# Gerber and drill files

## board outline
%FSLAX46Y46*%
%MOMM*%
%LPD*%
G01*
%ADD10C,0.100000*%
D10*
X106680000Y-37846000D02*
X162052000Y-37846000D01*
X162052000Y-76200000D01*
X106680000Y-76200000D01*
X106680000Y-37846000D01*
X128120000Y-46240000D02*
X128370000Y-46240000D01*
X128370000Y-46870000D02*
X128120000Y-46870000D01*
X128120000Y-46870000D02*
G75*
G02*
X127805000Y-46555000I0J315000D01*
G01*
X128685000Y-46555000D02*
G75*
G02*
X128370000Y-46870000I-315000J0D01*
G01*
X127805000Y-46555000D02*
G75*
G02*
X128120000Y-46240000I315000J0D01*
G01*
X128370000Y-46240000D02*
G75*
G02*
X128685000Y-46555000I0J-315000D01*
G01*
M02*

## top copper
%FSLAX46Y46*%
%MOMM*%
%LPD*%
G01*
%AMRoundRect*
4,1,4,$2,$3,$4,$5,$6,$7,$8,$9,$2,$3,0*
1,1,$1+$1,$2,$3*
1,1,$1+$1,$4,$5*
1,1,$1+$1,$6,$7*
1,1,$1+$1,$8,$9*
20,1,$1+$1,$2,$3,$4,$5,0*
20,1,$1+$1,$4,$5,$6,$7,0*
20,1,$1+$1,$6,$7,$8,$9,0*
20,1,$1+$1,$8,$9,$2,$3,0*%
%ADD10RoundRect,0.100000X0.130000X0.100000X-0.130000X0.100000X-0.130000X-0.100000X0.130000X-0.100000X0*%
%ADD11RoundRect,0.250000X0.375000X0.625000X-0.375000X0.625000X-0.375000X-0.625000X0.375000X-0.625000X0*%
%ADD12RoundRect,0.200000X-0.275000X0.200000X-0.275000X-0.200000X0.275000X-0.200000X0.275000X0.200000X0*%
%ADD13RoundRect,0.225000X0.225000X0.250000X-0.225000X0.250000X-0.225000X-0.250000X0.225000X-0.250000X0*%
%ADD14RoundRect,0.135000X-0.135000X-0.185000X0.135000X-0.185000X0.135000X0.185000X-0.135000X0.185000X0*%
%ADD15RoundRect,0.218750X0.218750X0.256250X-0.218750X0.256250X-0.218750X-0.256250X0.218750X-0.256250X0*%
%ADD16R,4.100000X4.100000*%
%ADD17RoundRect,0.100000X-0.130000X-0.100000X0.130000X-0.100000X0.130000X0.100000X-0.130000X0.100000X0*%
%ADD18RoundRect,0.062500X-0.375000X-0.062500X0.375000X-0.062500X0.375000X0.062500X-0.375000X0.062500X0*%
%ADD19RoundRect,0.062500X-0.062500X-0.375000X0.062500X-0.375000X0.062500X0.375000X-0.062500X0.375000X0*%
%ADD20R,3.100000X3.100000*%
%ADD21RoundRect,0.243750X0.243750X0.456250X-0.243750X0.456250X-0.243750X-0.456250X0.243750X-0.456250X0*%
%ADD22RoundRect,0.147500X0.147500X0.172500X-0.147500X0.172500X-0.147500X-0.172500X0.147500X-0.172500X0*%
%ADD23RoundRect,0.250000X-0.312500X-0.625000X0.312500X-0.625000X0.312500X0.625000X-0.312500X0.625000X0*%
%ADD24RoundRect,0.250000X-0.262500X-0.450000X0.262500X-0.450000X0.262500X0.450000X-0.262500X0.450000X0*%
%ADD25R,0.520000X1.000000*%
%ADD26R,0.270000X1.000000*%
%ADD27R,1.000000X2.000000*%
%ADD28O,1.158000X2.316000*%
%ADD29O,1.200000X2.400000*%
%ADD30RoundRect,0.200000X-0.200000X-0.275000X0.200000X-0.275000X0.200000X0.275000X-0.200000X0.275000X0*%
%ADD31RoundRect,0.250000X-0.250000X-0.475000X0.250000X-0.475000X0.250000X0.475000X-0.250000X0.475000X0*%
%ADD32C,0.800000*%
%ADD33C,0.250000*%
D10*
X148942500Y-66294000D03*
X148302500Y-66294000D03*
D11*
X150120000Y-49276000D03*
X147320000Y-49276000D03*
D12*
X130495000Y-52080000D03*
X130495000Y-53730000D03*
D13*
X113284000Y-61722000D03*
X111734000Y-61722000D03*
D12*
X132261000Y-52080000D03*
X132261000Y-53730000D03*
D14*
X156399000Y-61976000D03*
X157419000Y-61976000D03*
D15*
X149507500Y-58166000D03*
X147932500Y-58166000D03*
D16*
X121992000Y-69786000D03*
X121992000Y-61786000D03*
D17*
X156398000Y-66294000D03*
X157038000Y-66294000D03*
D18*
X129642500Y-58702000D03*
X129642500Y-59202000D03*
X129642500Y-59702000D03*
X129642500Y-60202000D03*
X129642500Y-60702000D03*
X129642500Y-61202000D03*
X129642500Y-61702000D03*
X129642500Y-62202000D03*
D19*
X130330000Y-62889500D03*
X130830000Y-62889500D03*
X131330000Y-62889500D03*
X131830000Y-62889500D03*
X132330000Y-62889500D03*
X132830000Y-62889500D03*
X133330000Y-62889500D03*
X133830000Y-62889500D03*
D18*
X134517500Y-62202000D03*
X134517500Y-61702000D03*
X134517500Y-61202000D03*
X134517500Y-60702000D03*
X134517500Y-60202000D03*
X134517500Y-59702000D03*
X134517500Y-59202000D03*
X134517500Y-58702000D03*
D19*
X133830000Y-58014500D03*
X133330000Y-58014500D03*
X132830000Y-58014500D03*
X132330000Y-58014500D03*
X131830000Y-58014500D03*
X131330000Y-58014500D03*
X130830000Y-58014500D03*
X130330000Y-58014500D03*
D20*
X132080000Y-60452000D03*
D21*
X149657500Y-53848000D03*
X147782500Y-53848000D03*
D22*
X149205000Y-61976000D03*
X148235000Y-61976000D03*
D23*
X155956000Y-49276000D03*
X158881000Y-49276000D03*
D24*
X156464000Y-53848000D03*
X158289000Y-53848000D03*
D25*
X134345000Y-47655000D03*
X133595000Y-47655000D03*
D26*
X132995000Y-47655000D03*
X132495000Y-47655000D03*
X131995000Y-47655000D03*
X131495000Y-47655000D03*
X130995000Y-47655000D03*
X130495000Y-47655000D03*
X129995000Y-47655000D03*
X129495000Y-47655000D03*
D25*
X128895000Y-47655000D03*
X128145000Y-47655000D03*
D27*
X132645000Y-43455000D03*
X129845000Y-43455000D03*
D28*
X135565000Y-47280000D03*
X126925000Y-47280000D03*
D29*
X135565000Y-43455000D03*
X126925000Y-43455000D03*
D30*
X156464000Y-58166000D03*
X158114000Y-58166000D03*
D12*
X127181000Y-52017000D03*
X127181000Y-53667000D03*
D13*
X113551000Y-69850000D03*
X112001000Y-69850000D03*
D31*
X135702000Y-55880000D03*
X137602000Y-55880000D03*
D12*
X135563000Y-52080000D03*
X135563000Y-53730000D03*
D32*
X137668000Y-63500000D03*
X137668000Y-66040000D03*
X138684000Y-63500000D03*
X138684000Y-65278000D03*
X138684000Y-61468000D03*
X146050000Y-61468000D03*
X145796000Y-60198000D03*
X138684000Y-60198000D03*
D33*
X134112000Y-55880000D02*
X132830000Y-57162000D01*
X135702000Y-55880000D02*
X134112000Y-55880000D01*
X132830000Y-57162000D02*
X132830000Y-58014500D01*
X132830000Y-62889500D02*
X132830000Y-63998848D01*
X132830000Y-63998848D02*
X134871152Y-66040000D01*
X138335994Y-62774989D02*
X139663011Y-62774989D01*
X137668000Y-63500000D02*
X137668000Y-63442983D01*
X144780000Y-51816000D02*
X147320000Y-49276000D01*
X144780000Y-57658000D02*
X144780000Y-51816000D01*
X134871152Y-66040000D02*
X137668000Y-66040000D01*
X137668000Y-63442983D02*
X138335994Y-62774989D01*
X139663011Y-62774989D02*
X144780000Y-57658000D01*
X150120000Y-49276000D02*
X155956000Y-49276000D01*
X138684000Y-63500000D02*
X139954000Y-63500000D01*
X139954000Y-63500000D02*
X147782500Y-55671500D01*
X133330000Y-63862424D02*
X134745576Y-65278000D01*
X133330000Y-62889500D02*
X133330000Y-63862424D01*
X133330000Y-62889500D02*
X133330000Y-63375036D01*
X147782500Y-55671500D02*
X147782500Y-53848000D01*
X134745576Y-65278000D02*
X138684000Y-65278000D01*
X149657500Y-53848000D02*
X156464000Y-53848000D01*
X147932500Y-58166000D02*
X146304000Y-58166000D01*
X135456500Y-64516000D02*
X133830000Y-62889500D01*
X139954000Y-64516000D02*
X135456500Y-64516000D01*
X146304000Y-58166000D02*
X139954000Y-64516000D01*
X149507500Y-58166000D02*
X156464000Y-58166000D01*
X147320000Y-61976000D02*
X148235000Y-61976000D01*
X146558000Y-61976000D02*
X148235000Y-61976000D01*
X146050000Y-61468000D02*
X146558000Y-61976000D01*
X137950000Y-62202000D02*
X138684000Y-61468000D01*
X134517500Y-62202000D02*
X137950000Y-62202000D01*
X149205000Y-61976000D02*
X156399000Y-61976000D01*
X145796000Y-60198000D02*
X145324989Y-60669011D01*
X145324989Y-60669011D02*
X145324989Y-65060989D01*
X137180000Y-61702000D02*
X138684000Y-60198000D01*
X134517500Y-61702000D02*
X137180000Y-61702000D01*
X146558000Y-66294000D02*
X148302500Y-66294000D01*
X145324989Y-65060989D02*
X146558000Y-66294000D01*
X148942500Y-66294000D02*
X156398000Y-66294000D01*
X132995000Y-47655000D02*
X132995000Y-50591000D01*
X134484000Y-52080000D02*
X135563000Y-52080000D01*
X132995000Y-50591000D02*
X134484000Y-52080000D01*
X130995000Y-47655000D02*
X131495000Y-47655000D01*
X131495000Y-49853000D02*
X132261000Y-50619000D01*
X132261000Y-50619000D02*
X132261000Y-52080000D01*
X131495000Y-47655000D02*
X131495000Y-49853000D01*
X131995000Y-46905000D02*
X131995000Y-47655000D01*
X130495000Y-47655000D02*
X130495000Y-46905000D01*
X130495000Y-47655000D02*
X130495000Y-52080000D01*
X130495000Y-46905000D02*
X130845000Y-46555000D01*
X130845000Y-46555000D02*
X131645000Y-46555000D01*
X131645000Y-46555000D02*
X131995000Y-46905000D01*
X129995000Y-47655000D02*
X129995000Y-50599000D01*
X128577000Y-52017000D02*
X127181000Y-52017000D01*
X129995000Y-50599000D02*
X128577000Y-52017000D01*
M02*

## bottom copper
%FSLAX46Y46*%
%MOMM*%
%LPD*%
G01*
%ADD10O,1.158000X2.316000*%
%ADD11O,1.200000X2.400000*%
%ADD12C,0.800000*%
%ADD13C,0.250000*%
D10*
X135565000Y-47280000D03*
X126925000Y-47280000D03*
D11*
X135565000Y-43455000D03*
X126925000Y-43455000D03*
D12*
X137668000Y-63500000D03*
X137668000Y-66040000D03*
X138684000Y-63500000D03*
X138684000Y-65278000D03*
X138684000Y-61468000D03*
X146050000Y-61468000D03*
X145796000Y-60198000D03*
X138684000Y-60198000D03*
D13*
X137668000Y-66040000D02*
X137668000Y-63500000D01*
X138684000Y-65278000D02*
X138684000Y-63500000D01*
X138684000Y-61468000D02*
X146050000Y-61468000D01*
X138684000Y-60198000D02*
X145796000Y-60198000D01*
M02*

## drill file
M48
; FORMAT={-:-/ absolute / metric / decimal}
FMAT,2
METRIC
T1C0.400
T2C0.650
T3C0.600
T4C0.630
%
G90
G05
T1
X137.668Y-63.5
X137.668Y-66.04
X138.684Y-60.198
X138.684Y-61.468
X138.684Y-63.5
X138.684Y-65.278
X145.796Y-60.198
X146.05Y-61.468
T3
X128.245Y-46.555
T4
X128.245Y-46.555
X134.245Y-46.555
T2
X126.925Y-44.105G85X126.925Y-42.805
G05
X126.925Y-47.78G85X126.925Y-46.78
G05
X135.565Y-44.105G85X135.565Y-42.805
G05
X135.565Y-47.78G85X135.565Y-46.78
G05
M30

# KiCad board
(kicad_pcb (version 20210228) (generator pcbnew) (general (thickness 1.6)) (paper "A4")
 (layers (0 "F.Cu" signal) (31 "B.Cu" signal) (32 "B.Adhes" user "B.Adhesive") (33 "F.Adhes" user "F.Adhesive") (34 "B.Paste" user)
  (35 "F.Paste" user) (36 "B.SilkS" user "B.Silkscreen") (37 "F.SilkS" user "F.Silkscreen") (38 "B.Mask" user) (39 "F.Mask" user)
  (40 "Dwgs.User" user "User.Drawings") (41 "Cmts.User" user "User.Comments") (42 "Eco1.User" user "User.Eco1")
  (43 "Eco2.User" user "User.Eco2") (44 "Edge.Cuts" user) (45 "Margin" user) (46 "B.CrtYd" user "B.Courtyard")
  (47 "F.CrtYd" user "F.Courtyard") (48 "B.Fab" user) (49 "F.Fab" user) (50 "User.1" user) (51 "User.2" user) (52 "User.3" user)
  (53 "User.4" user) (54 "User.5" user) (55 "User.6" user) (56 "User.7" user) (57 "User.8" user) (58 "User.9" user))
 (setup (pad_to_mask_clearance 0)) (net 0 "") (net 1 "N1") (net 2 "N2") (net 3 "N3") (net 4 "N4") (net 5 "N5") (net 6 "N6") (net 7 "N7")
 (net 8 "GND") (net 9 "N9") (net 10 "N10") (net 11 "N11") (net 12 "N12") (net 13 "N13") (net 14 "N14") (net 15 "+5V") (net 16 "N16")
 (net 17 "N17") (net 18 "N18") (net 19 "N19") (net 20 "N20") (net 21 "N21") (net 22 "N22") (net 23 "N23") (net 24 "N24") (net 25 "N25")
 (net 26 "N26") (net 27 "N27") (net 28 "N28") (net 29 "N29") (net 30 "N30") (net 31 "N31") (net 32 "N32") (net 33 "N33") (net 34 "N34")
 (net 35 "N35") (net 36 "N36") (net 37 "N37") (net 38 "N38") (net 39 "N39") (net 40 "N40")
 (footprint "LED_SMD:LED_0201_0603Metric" (layer "F.Cu") (at 148.6225 66.294 180)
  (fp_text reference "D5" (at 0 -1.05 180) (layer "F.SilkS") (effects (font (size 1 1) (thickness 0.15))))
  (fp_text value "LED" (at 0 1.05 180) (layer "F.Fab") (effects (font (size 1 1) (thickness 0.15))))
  (pad "" smd roundrect (at 0.345 0 180) (locked) (size 0.318 0.36) (layers "F.Paste") (roundrect_rratio 0.25))
  (pad "" smd roundrect (at -0.345 0 180) (locked) (size 0.318 0.36) (layers "F.Paste") (roundrect_rratio 0.25))
  (pad "1" smd roundrect (at -0.32 0 180) (locked) (size 0.46 0.4) (layers "F.Cu" "F.Mask") (roundrect_rratio 0.25) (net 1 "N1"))
  (pad "2" smd roundrect (at 0.32 0 180) (locked) (size 0.46 0.4) (layers "F.Cu" "F.Mask") (roundrect_rratio 0.25) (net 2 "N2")))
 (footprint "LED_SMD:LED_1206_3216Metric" (layer "F.Cu") (at 148.72 49.276 180)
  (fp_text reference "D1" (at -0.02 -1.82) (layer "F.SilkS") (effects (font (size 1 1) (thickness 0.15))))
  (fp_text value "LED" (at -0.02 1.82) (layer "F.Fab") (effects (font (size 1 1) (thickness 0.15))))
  (pad "1" smd roundrect (at -1.4 0 180) (locked) (size 1.25 1.75) (layers "F.Cu" "F.Paste" "F.Mask") (roundrect_rratio 0.2) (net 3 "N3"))
  (pad "2" smd roundrect (at 1.4 0 180) (locked) (size 1.25 1.75) (layers "F.Cu" "F.Paste" "F.Mask") (roundrect_rratio 0.2) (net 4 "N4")))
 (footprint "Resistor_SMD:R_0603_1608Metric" (layer "F.Cu") (at 130.495 52.905 -90)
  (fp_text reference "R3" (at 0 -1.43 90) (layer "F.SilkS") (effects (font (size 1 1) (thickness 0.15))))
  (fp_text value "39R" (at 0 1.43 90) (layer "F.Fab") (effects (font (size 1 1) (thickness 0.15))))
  (pad "1" smd roundrect (at -0.825 0 270) (locked) (size 0.8 0.95) (layers "F.Cu" "F.Paste" "F.Mask") (roundrect_rratio 0.25) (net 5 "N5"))
  (pad "2" smd roundrect (at 0.825 0 270) (locked) (size 0.8 0.95) (layers "F.Cu" "F.Paste" "F.Mask") (roundrect_rratio 0.25) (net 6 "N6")))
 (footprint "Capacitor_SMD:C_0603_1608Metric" (layer "F.Cu") (at 112.509 61.722 180)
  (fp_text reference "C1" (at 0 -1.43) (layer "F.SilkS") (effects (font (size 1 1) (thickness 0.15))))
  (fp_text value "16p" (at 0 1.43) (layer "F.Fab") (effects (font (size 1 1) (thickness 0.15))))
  (pad "1" smd roundrect (at -0.775 0 180) (locked) (size 0.9 0.95) (layers "F.Cu" "F.Paste" "F.Mask") (roundrect_rratio 0.25) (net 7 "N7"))
  (pad "2" smd roundrect (at 0.775 0 180) (locked) (size 0.9 0.95) (layers "F.Cu" "F.Paste" "F.Mask") (roundrect_rratio 0.25) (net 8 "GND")))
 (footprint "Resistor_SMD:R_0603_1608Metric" (layer "F.Cu") (at 132.261 52.905 -90)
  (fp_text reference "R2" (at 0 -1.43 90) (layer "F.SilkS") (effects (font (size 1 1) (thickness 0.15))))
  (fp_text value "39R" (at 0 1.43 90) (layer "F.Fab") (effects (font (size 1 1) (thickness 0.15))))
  (pad "1" smd roundrect (at -0.825 0 270) (locked) (size 0.8 0.95) (layers "F.Cu" "F.Paste" "F.Mask") (roundrect_rratio 0.25) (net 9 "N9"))
  (pad "2" smd roundrect (at 0.825 0 270) (locked) (size 0.8 0.95) (layers "F.Cu" "F.Paste" "F.Mask") (roundrect_rratio 0.25) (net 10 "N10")))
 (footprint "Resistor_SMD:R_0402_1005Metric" (layer "F.Cu") (at 156.909 61.976)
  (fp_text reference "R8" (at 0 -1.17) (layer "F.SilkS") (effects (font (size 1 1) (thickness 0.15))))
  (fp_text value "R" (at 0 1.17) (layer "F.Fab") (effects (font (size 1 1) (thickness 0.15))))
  (pad "1" smd roundrect (at -0.51 0) (locked) (size 0.54 0.64) (layers "F.Cu" "F.Paste" "F.Mask") (roundrect_rratio 0.25) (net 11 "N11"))
  (pad "2" smd roundrect (at 0.51 0) (locked) (size 0.54 0.64) (layers "F.Cu" "F.Paste" "F.Mask") (roundrect_rratio 0.25) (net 8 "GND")))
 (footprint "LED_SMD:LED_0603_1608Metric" (layer "F.Cu") (at 148.72 58.166 180)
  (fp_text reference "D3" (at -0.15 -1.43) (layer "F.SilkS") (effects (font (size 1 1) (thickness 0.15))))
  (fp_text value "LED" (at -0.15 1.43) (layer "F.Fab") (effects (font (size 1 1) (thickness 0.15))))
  (pad "1" smd roundrect (at -0.7875 0 180) (locked) (size 0.875 0.95) (layers "F.Cu" "F.Paste" "F.Mask") (roundrect_rratio 0.25)
   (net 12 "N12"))
  (pad "2" smd roundrect (at 0.7875 0 180) (locked) (size 0.875 0.95) (layers "F.Cu" "F.Paste" "F.Mask") (roundrect_rratio 0.25)
   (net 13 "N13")))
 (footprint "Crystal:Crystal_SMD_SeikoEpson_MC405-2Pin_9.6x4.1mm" (layer "F.Cu") (at 121.992 65.786 90)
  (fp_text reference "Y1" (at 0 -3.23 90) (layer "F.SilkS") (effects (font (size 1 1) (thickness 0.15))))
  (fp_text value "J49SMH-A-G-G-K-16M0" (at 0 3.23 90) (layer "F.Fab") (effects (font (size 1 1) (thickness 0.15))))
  (pad "1" smd rect (at -4 0 90) (locked) (size 4.1 4.1) (layers "F.Cu" "F.Paste" "F.Mask") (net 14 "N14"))
  (pad "2" smd rect (at 4 0 90) (locked) (size 4.1 4.1) (layers "F.Cu" "F.Paste" "F.Mask") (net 7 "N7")))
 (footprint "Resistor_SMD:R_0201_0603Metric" (layer "F.Cu") (at 156.718 66.294)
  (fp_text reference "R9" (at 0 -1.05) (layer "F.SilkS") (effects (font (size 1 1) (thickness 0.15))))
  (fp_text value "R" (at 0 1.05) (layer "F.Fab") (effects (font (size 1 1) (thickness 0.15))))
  (pad "" smd roundrect (at -0.345 0) (locked) (size 0.318 0.36) (layers "F.Paste") (roundrect_rratio 0.25))
  (pad "" smd roundrect (at 0.345 0) (locked) (size 0.318 0.36) (layers "F.Paste") (roundrect_rratio 0.25))
  (pad "1" smd roundrect (at -0.32 0) (locked) (size 0.46 0.4) (layers "F.Cu" "F.Mask") (roundrect_rratio 0.25) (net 1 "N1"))
  (pad "2" smd roundrect (at 0.32 0) (locked) (size 0.46 0.4) (layers "F.Cu" "F.Mask") (roundrect_rratio 0.25) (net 8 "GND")))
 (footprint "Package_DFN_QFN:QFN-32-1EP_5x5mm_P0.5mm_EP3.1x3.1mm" (layer "F.Cu") (at 132.08 60.452)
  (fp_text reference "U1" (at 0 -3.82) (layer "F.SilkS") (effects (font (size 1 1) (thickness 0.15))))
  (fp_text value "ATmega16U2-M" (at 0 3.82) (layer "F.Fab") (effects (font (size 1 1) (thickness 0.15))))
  (pad "" smd roundrect (at 1.03 -1.03) (locked) (size 0.83 0.83) (layers "F.Paste") (roundrect_rratio 0.25))
  (pad "" smd roundrect (at 0 -1.03) (locked) (size 0.83 0.83) (layers "F.Paste") (roundrect_rratio 0.25))
  (pad "" smd roundrect (at 0 1.03) (locked) (size 0.83 0.83) (layers "F.Paste") (roundrect_rratio 0.25))
  (pad "" smd roundrect (at 0 0) (locked) (size 0.83 0.83) (layers "F.Paste") (roundrect_rratio 0.25))
  (pad "" smd roundrect (at 1.03 1.03) (locked) (size 0.83 0.83) (layers "F.Paste") (roundrect_rratio 0.25))
  (pad "" smd roundrect (at 1.03 0) (locked) (size 0.83 0.83) (layers "F.Paste") (roundrect_rratio 0.25))
  (pad "" smd roundrect (at -1.03 -1.03) (locked) (size 0.83 0.83) (layers "F.Paste") (roundrect_rratio 0.25))
  (pad "" smd roundrect (at -1.03 1.03) (locked) (size 0.83 0.83) (layers "F.Paste") (roundrect_rratio 0.25))
  (pad "" smd roundrect (at -1.03 0) (locked) (size 0.83 0.83) (layers "F.Paste") (roundrect_rratio 0.25))
  (pad "1" smd roundrect (at -2.4375 -1.75) (locked) (size 0.875 0.25) (layers "F.Cu" "F.Paste" "F.Mask") (roundrect_rratio 0.25)
   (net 7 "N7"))
  (pad "2" smd roundrect (at -2.4375 -1.25) (locked) (size 0.875 0.25) (layers "F.Cu" "F.Paste" "F.Mask") (roundrect_rratio 0.25)
   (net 14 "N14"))
  (pad "3" smd roundrect (at -2.4375 -0.75) (locked) (size 0.875 0.25) (layers "F.Cu" "F.Paste" "F.Mask") (roundrect_rratio 0.25)
   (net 8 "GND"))
  (pad "4" smd roundrect (at -2.4375 -0.25) (locked) (size 0.875 0.25) (layers "F.Cu" "F.Paste" "F.Mask") (roundrect_rratio 0.25)
   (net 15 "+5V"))
  (pad "5" smd roundrect (at -2.4375 0.25) (locked) (size 0.875 0.25) (layers "F.Cu" "F.Paste" "F.Mask") (roundrect_rratio 0.25)
   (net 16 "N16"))
  (pad "6" smd roundrect (at -2.4375 0.75) (locked) (size 0.875 0.25) (layers "F.Cu" "F.Paste" "F.Mask") (roundrect_rratio 0.25)
   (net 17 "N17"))
  (pad "7" smd roundrect (at -2.4375 1.25) (locked) (size 0.875 0.25) (layers "F.Cu" "F.Paste" "F.Mask") (roundrect_rratio 0.25)
   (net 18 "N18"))
  (pad "8" smd roundrect (at -2.4375 1.75) (locked) (size 0.875 0.25) (layers "F.Cu" "F.Paste" "F.Mask") (roundrect_rratio 0.25)
   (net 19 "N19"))
  (pad "9" smd roundrect (at -1.75 2.4375) (locked) (size 0.25 0.875) (layers "F.Cu" "F.Paste" "F.Mask") (roundrect_rratio 0.25)
   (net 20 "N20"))
  (pad "10" smd roundrect (at -1.25 2.4375) (locked) (size 0.25 0.875) (layers "F.Cu" "F.Paste" "F.Mask") (roundrect_rratio 0.25)
   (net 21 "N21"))
  (pad "11" smd roundrect (at -0.75 2.4375) (locked) (size 0.25 0.875) (layers "F.Cu" "F.Paste" "F.Mask") (roundrect_rratio 0.25)
   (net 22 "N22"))
  (pad "12" smd roundrect (at -0.25 2.4375) (locked) (size 0.25 0.875) (layers "F.Cu" "F.Paste" "F.Mask") (roundrect_rratio 0.25)
   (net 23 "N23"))
  (pad "13" smd roundrect (at 0.25 2.4375) (locked) (size 0.25 0.875) (layers "F.Cu" "F.Paste" "F.Mask") (roundrect_rratio 0.25)
   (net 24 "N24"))
  (pad "14" smd roundrect (at 0.75 2.4375) (locked) (size 0.25 0.875) (layers "F.Cu" "F.Paste" "F.Mask") (roundrect_rratio 0.25)
   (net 4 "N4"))
  (pad "15" smd roundrect (at 1.25 2.4375) (locked) (size 0.25 0.875) (layers "F.Cu" "F.Paste" "F.Mask") (roundrect_rratio 0.25)
   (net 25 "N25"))
  (pad "16" smd roundrect (at 1.75 2.4375) (locked) (size 0.25 0.875) (layers "F.Cu" "F.Paste" "F.Mask") (roundrect_rratio 0.25)
   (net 13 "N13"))
  (pad "17" smd roundrect (at 2.4375 1.75) (locked) (size 0.875 0.25) (layers "F.Cu" "F.Paste" "F.Mask") (roundrect_rratio 0.25)
   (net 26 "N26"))
  (pad "18" smd roundrect (at 2.4375 1.25) (locked) (size 0.875 0.25) (layers "F.Cu" "F.Paste" "F.Mask") (roundrect_rratio 0.25)
   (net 2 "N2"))
  (pad "19" smd roundrect (at 2.4375 0.75) (locked) (size 0.875 0.25) (layers "F.Cu" "F.Paste" "F.Mask") (roundrect_rratio 0.25)
   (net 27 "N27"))
  (pad "20" smd roundrect (at 2.4375 0.25) (locked) (size 0.875 0.25) (layers "F.Cu" "F.Paste" "F.Mask") (roundrect_rratio 0.25)
   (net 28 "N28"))
  (pad "21" smd roundrect (at 2.4375 -0.25) (locked) (size 0.875 0.25) (layers "F.Cu" "F.Paste" "F.Mask") (roundrect_rratio 0.25)
   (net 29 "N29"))
  (pad "22" smd roundrect (at 2.4375 -0.75) (locked) (size 0.875 0.25) (layers "F.Cu" "F.Paste" "F.Mask") (roundrect_rratio 0.25)
   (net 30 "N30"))
  (pad "23" smd roundrect (at 2.4375 -1.25) (locked) (size 0.875 0.25) (layers "F.Cu" "F.Paste" "F.Mask") (roundrect_rratio 0.25)
   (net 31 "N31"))
  (pad "24" smd roundrect (at 2.4375 -1.75) (locked) (size 0.875 0.25) (layers "F.Cu" "F.Paste" "F.Mask") (roundrect_rratio 0.25)
   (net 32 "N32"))
  (pad "25" smd roundrect (at 1.75 -2.4375) (locked) (size 0.25 0.875) (layers "F.Cu" "F.Paste" "F.Mask") (roundrect_rratio 0.25)
   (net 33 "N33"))
  (pad "26" smd roundrect (at 1.25 -2.4375) (locked) (size 0.25 0.875) (layers "F.Cu" "F.Paste" "F.Mask") (roundrect_rratio 0.25)
   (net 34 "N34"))
  (pad "27" smd roundrect (at 0.75 -2.4375) (locked) (size 0.25 0.875) (layers "F.Cu" "F.Paste" "F.Mask") (roundrect_rratio 0.25)
   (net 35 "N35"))
  (pad "28" smd roundrect (at 0.25 -2.4375) (locked) (size 0.25 0.875) (layers "F.Cu" "F.Paste" "F.Mask") (roundrect_rratio 0.25)
   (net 8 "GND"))
  (pad "29" smd roundrect (at -0.25 -2.4375) (locked) (size 0.25 0.875) (layers "F.Cu" "F.Paste" "F.Mask") (roundrect_rratio 0.25)
   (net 10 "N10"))
  (pad "30" smd roundrect (at -0.75 -2.4375) (locked) (size 0.25 0.875) (layers "F.Cu" "F.Paste" "F.Mask") (roundrect_rratio 0.25)
   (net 6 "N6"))
  (pad "31" smd roundrect (at -1.25 -2.4375) (locked) (size 0.25 0.875) (layers "F.Cu" "F.Paste" "F.Mask") (roundrect_rratio 0.25)
   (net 15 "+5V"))
  (pad "32" smd roundrect (at -1.75 -2.4375) (locked) (size 0.25 0.875) (layers "F.Cu" "F.Paste" "F.Mask") (roundrect_rratio 0.25)
   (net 15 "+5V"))
  (pad "33" smd rect (at 0 0) (locked) (size 3.1 3.1) (layers "F.Cu" "F.Mask") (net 8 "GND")))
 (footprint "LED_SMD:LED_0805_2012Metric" (layer "F.Cu") (at 148.72 53.848 180)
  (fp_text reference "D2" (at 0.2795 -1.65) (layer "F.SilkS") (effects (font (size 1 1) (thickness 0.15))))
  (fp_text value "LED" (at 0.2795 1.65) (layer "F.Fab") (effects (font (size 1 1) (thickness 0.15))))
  (pad "1" smd roundrect (at -0.9375 0 180) (locked) (size 0.975 1.4) (layers "F.Cu" "F.Paste" "F.Mask") (roundrect_rratio 0.25)
   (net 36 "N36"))
  (pad "2" smd roundrect (at 0.9375 0 180) (locked) (size 0.975 1.4) (layers "F.Cu" "F.Paste" "F.Mask") (roundrect_rratio 0.25)
   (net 25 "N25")))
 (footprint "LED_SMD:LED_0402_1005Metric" (layer "F.Cu") (at 148.72 61.976 180)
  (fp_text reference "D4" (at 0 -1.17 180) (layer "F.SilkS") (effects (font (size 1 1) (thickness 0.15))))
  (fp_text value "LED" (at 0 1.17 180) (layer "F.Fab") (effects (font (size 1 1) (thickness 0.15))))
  (pad "1" smd roundrect (at -0.485 0 180) (locked) (size 0.59 0.64) (layers "F.Cu" "F.Paste" "F.Mask") (roundrect_rratio 0.25)
   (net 11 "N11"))
  (pad "2" smd roundrect (at 0.485 0 180) (locked) (size 0.59 0.64) (layers "F.Cu" "F.Paste" "F.Mask") (roundrect_rratio 0.25)
   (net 26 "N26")))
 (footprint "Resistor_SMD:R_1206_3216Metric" (layer "F.Cu") (at 157.4185 49.276)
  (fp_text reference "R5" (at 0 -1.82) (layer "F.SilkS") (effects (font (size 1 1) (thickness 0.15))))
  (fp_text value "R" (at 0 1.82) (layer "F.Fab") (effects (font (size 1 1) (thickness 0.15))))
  (pad "1" smd roundrect (at -1.4625 0) (locked) (size 1.125 1.75) (layers "F.Cu" "F.Paste" "F.Mask") (roundrect_rratio 0.222222)
   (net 3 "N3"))
  (pad "2" smd roundrect (at 1.4625 0) (locked) (size 1.125 1.75) (layers "F.Cu" "F.Paste" "F.Mask") (roundrect_rratio 0.222222)
   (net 8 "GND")))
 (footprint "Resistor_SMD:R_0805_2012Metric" (layer "F.Cu") (at 157.3765 53.848)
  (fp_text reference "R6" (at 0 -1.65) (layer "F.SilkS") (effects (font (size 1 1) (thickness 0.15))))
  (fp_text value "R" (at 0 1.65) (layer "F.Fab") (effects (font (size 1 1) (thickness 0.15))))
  (pad "1" smd roundrect (at -0.9125 0) (locked) (size 1.025 1.4) (layers "F.Cu" "F.Paste" "F.Mask") (roundrect_rratio 0.243902)
   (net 36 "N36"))
  (pad "2" smd roundrect (at 0.9125 0) (locked) (size 1.025 1.4) (layers "F.Cu" "F.Paste" "F.Mask") (roundrect_rratio 0.243902)
   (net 8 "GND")))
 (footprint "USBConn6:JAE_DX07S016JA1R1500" (layer "F.Cu") (at 131.245 46.555 180)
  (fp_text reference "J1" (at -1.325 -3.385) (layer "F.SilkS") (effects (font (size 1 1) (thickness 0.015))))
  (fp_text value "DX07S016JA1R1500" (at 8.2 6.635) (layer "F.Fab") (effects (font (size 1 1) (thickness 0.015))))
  (fp_line (start 3.125 0.315) (end 2.875 0.315) (layer "Edge.Cuts") (width 0.1))
  (fp_line (start 2.875 -0.315) (end 3.125 -0.315) (layer "Edge.Cuts") (width 0.1))
  (fp_arc (start 3.125 0) (end 3.44 0) (angle -90) (layer "Edge.Cuts") (width 0.1))
  (fp_arc (start 2.875 0) (end 2.875 -0.315) (angle -90) (layer "Edge.Cuts") (width 0.1))
  (fp_arc (start 3.125 0) (end 3.125 0.315) (angle -90) (layer "Edge.Cuts") (width 0.1))
  (fp_arc (start 2.875 0) (end 2.56 0) (angle -90) (layer "Edge.Cuts") (width 0.1))
  (pad "1" smd rect (at -3.1 -1.1 180) (locked) (size 0.52 1) (layers "F.Cu" "F.Paste" "F.Mask") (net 8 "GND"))
  (pad "2" smd rect (at -2.35 -1.1 180) (locked) (size 0.52 1) (layers "F.Cu" "F.Paste" "F.Mask") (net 15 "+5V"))
  (pad "3" smd rect (at -1.75 -1.1 180) (locked) (size 0.27 1) (layers "F.Cu" "F.Paste" "F.Mask") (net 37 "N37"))
  (pad "4" smd rect (at -1.25 -1.1 180) (locked) (size 0.27 1) (layers "F.Cu" "F.Paste" "F.Mask") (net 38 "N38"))
  (pad "5" smd rect (at -0.75 -1.1 180) (locked) (size 0.27 1) (layers "F.Cu" "F.Paste" "F.Mask") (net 5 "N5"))
  (pad "6" smd rect (at -0.25 -1.1 180) (locked) (size 0.27 1) (layers "F.Cu" "F.Paste" "F.Mask") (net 9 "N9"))
  (pad "7" smd rect (at 0.25 -1.1 180) (locked) (size 0.27 1) (layers "F.Cu" "F.Paste" "F.Mask") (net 9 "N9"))
  (pad "8" smd rect (at 0.75 -1.1 180) (locked) (size 0.27 1) (layers "F.Cu" "F.Paste" "F.Mask") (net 5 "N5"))
  (pad "9" smd rect (at 1.25 -1.1 180) (locked) (size 0.27 1) (layers "F.Cu" "F.Paste" "F.Mask") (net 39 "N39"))
  (pad "10" smd rect (at 1.75 -1.1 180) (locked) (size 0.27 1) (layers "F.Cu" "F.Paste" "F.Mask") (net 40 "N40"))
  (pad "11" smd rect (at 2.35 -1.1 180) (locked) (size 0.52 1) (layers "F.Cu" "F.Paste" "F.Mask") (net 15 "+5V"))
  (pad "12" smd rect (at 3.1 -1.1 180) (locked) (size 0.52 1) (layers "F.Cu" "F.Paste" "F.Mask") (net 8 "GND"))
  (pad "None" np_thru_hole circle (at 3 0 180) (locked) (size 0.63 0.63) (drill 0.63) (layers *.Cu *.Mask))
  (pad "None" np_thru_hole circle (at 3 0 180) (locked) (size 0.6 0.6) (drill 0.6) (layers *.Cu *.Mask))
  (pad "None" np_thru_hole circle (at -3 0 180) (locked) (size 0.63 0.63) (drill 0.63) (layers *.Cu *.Mask))
  (pad "S1" smd rect (at -1.4 3.1 180) (locked) (size 1 2) (layers "F.Cu" "F.Paste" "F.Mask") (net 8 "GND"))
  (pad "S2" smd rect (at 1.4 3.1 180) (locked) (size 1 2) (layers "F.Cu" "F.Paste" "F.Mask") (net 8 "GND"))
  (pad "S3" thru_hole oval (at -4.32 -0.725 180) (locked) (size 1.158 2.316) (drill oval 0.65 1.65) (layers *.Cu *.Mask) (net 8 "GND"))
  (pad "S4" thru_hole oval (at 4.32 -0.725 180) (locked) (size 1.158 2.316) (drill oval 0.65 1.65) (layers *.Cu *.Mask) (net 8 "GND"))
  (pad "S5" thru_hole oval (at -4.32 3.1 180) (locked) (size 1.2 2.4) (drill oval 0.65 1.95) (layers *.Cu *.Mask) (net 8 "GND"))
  (pad "S6" thru_hole oval (at 4.32 3.1 180) (locked) (size 1.2 2.4) (drill oval 0.65 1.95) (layers *.Cu *.Mask) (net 8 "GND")))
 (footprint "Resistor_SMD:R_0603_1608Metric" (layer "F.Cu") (at 157.289 58.166)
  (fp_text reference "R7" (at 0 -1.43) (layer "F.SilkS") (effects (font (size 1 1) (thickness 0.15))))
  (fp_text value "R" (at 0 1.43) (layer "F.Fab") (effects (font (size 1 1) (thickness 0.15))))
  (pad "1" smd roundrect (at -0.825 0) (locked) (size 0.8 0.95) (layers "F.Cu" "F.Paste" "F.Mask") (roundrect_rratio 0.25) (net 12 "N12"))
  (pad "2" smd roundrect (at 0.825 0) (locked) (size 0.8 0.95) (layers "F.Cu" "F.Paste" "F.Mask") (roundrect_rratio 0.25) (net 8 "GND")))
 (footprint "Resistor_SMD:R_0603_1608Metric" (layer "F.Cu") (at 127.181 52.842 -90)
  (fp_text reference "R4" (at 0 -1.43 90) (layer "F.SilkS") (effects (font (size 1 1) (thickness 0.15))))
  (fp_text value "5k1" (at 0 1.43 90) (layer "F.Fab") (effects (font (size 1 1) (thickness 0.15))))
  (pad "1" smd roundrect (at -0.825 0 270) (locked) (size 0.8 0.95) (layers "F.Cu" "F.Paste" "F.Mask") (roundrect_rratio 0.25)
   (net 39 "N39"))
  (pad "2" smd roundrect (at 0.825 0 270) (locked) (size 0.8 0.95) (layers "F.Cu" "F.Paste" "F.Mask") (roundrect_rratio 0.25) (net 8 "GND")))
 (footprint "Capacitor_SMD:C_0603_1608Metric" (layer "F.Cu") (at 112.776 69.85 180)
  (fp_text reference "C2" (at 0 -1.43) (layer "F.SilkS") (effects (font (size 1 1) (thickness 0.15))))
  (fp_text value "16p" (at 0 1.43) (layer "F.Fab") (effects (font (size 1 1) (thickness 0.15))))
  (pad "1" smd roundrect (at -0.775 0 180) (locked) (size 0.9 0.95) (layers "F.Cu" "F.Paste" "F.Mask") (roundrect_rratio 0.25)
   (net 14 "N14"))
  (pad "2" smd roundrect (at 0.775 0 180) (locked) (size 0.9 0.95) (layers "F.Cu" "F.Paste" "F.Mask") (roundrect_rratio 0.25) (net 8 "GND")))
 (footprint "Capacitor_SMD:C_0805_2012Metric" (layer "F.Cu") (at 136.652 55.88)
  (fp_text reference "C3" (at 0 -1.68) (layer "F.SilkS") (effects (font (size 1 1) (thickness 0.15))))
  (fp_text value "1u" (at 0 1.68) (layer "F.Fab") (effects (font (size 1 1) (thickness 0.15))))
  (pad "1" smd roundrect (at -0.95 0) (locked) (size 1 1.45) (layers "F.Cu" "F.Paste" "F.Mask") (roundrect_rratio 0.25) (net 35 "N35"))
  (pad "2" smd roundrect (at 0.95 0) (locked) (size 1 1.45) (layers "F.Cu" "F.Paste" "F.Mask") (roundrect_rratio 0.25) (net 8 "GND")))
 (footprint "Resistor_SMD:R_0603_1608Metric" (layer "F.Cu") (at 135.563 52.905 -90)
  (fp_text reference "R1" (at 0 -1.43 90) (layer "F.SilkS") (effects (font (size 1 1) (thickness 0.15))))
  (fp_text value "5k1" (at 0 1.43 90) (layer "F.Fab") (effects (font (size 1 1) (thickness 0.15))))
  (pad "1" smd roundrect (at -0.825 0 270) (locked) (size 0.8 0.95) (layers "F.Cu" "F.Paste" "F.Mask") (roundrect_rratio 0.25)
   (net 37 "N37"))
  (pad "2" smd roundrect (at 0.825 0 270) (locked) (size 0.8 0.95) (layers "F.Cu" "F.Paste" "F.Mask") (roundrect_rratio 0.25) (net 8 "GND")))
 (gr_rect (start 106.68 37.846) (end 162.052 76.2) (layer "Edge.Cuts") (width 0.1) (fill none))
 (segment (start 134.112 55.88) (end 132.83 57.162) (width 0.25) (layer "F.Cu") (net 35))
 (segment (start 135.702 55.88) (end 134.112 55.88) (width 0.25) (layer "F.Cu") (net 35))
 (segment (start 132.83 57.162) (end 132.83 58.0145) (width 0.25) (layer "F.Cu") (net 35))
 (segment (start 132.83 62.8895) (end 132.83 63.998848) (width 0.25) (layer "F.Cu") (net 4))
 (segment (start 132.83 63.998848) (end 134.871152 66.04) (width 0.25) (layer "F.Cu") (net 4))
 (segment (start 138.335994 62.774989) (end 139.663011 62.774989) (width 0.25) (layer "F.Cu") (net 4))
 (segment (start 137.668 63.5) (end 137.668 63.442983) (width 0.25) (layer "F.Cu") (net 4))
 (segment (start 144.78 51.816) (end 147.32 49.276) (width 0.25) (layer "F.Cu") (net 4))
 (segment (start 144.78 57.658) (end 144.78 51.816) (width 0.25) (layer "F.Cu") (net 4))
 (segment (start 134.871152 66.04) (end 137.668 66.04) (width 0.25) (layer "F.Cu") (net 4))
 (segment (start 137.668 63.442983) (end 138.335994 62.774989) (width 0.25) (layer "F.Cu") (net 4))
 (segment (start 139.663011 62.774989) (end 144.78 57.658) (width 0.25) (layer "F.Cu") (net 4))
 (via (at 137.668 63.5) (size 0.8) (drill 0.4) (layers "F.Cu" "B.Cu") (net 4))
 (via (at 137.668 66.04) (size 0.8) (drill 0.4) (layers "F.Cu" "B.Cu") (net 4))
 (segment (start 137.668 66.04) (end 137.668 63.5) (width 0.25) (layer "B.Cu") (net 4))
 (segment (start 150.12 49.276) (end 155.956 49.276) (width 0.25) (layer "F.Cu") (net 3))
 (segment (start 138.684 63.5) (end 139.954 63.5) (width 0.25) (layer "F.Cu") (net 25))
 (segment (start 139.954 63.5) (end 147.7825 55.6715) (width 0.25) (layer "F.Cu") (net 25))
 (segment (start 133.33 63.862424) (end 134.745576 65.278) (width 0.25) (layer "F.Cu") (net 25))
 (segment (start 133.33 62.8895) (end 133.33 63.862424) (width 0.25) (layer "F.Cu") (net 25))
 (segment (start 133.33 62.8895) (end 133.33 63.375036) (width 0.25) (layer "F.Cu") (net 25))
 (segment (start 147.7825 55.6715) (end 147.7825 53.848) (width 0.25) (layer "F.Cu") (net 25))
 (segment (start 134.745576 65.278) (end 138.684 65.278) (width 0.25) (layer "F.Cu") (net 25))
 (via (at 138.684 63.5) (size 0.8) (drill 0.4) (layers "F.Cu" "B.Cu") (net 25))
 (via (at 138.684 65.278) (size 0.8) (drill 0.4) (layers "F.Cu" "B.Cu") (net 25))
 (segment (start 138.684 65.278) (end 138.684 63.5) (width 0.25) (layer "B.Cu") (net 25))
 (segment (start 149.6575 53.848) (end 156.464 53.848) (width 0.25) (layer "F.Cu") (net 36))
 (segment (start 147.9325 58.166) (end 146.304 58.166) (width 0.25) (layer "F.Cu") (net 13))
 (segment (start 135.4565 64.516) (end 133.83 62.8895) (width 0.25) (layer "F.Cu") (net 13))
 (segment (start 139.954 64.516) (end 135.4565 64.516) (width 0.25) (layer "F.Cu") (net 13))
 (segment (start 146.304 58.166) (end 139.954 64.516) (width 0.25) (layer "F.Cu") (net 13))
 (segment (start 149.5075 58.166) (end 156.464 58.166) (width 0.25) (layer "F.Cu") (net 12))
 (segment (start 147.32 61.976) (end 148.235 61.976) (width 0.25) (layer "F.Cu") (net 26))
 (segment (start 146.558 61.976) (end 148.235 61.976) (width 0.25) (layer "F.Cu") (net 26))
 (segment (start 146.05 61.468) (end 146.558 61.976) (width 0.25) (layer "F.Cu") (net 26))
 (segment (start 137.95 62.202) (end 138.684 61.468) (width 0.25) (layer "F.Cu") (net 26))
 (segment (start 134.5175 62.202) (end 137.95 62.202) (width 0.25) (layer "F.Cu") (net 26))
 (via (at 138.684 61.468) (size 0.8) (drill 0.4) (layers "F.Cu" "B.Cu") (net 26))
 (via (at 146.05 61.468) (size 0.8) (drill 0.4) (layers "F.Cu" "B.Cu") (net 26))
 (segment (start 138.684 61.468) (end 146.05 61.468) (width 0.25) (layer "B.Cu") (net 26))
 (segment (start 149.205 61.976) (end 156.399 61.976) (width 0.25) (layer "F.Cu") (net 11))
 (segment (start 145.796 60.198) (end 145.324989 60.669011) (width 0.25) (layer "F.Cu") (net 2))
 (segment (start 145.324989 60.669011) (end 145.324989 65.060989) (width 0.25) (layer "F.Cu") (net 2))
 (segment (start 137.18 61.702) (end 138.684 60.198) (width 0.25) (layer "F.Cu") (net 2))
 (segment (start 134.5175 61.702) (end 137.18 61.702) (width 0.25) (layer "F.Cu") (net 2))
 (segment (start 146.558 66.294) (end 148.3025 66.294) (width 0.25) (layer "F.Cu") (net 2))
 (segment (start 145.324989 65.060989) (end 146.558 66.294) (width 0.25) (layer "F.Cu") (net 2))
 (via (at 145.796 60.198) (size 0.8) (drill 0.4) (layers "F.Cu" "B.Cu") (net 2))
 (via (at 138.684 60.198) (size 0.8) (drill 0.4) (layers "F.Cu" "B.Cu") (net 2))
 (segment (start 138.684 60.198) (end 145.796 60.198) (width 0.25) (layer "B.Cu") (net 2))
 (segment (start 148.9425 66.294) (end 156.398 66.294) (width 0.25) (layer "F.Cu") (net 1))
 (segment (start 132.995 47.655) (end 132.995 50.591) (width 0.25) (layer "F.Cu") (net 37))
 (segment (start 134.484 52.08) (end 135.563 52.08) (width 0.25) (layer "F.Cu") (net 37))
 (segment (start 132.995 50.591) (end 134.484 52.08) (width 0.25) (layer "F.Cu") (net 37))
 (segment (start 130.995 47.655) (end 131.495 47.655) (width 0.25) (layer "F.Cu") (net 9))
 (segment (start 131.495 49.853) (end 132.261 50.619) (width 0.25) (layer "F.Cu") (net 9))
 (segment (start 132.261 50.619) (end 132.261 52.08) (width 0.25) (layer "F.Cu") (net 9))
 (segment (start 131.495 47.655) (end 131.495 49.853) (width 0.25) (layer "F.Cu") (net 9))
 (segment (start 131.995 46.905) (end 131.995 47.655) (width 0.25) (layer "F.Cu") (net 5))
 (segment (start 130.495 47.655) (end 130.495 46.905) (width 0.25) (layer "F.Cu") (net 5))
 (segment (start 130.495 47.655) (end 130.495 52.08) (width 0.25) (layer "F.Cu") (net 5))
 (segment (start 130.495 46.905) (end 130.845 46.555) (width 0.25) (layer "F.Cu") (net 5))
 (segment (start 130.845 46.555) (end 131.645 46.555) (width 0.25) (layer "F.Cu") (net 5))
 (segment (start 131.645 46.555) (end 131.995 46.905) (width 0.25) (layer "F.Cu") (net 5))
 (segment (start 129.995 47.655) (end 129.995 50.599) (width 0.25) (layer "F.Cu") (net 39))
 (segment (start 128.577 52.017) (end 127.181 52.017) (width 0.25) (layer "F.Cu") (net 39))
 (segment (start 129.995 50.599) (end 128.577 52.017) (width 0.25) (layer "F.Cu") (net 39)))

